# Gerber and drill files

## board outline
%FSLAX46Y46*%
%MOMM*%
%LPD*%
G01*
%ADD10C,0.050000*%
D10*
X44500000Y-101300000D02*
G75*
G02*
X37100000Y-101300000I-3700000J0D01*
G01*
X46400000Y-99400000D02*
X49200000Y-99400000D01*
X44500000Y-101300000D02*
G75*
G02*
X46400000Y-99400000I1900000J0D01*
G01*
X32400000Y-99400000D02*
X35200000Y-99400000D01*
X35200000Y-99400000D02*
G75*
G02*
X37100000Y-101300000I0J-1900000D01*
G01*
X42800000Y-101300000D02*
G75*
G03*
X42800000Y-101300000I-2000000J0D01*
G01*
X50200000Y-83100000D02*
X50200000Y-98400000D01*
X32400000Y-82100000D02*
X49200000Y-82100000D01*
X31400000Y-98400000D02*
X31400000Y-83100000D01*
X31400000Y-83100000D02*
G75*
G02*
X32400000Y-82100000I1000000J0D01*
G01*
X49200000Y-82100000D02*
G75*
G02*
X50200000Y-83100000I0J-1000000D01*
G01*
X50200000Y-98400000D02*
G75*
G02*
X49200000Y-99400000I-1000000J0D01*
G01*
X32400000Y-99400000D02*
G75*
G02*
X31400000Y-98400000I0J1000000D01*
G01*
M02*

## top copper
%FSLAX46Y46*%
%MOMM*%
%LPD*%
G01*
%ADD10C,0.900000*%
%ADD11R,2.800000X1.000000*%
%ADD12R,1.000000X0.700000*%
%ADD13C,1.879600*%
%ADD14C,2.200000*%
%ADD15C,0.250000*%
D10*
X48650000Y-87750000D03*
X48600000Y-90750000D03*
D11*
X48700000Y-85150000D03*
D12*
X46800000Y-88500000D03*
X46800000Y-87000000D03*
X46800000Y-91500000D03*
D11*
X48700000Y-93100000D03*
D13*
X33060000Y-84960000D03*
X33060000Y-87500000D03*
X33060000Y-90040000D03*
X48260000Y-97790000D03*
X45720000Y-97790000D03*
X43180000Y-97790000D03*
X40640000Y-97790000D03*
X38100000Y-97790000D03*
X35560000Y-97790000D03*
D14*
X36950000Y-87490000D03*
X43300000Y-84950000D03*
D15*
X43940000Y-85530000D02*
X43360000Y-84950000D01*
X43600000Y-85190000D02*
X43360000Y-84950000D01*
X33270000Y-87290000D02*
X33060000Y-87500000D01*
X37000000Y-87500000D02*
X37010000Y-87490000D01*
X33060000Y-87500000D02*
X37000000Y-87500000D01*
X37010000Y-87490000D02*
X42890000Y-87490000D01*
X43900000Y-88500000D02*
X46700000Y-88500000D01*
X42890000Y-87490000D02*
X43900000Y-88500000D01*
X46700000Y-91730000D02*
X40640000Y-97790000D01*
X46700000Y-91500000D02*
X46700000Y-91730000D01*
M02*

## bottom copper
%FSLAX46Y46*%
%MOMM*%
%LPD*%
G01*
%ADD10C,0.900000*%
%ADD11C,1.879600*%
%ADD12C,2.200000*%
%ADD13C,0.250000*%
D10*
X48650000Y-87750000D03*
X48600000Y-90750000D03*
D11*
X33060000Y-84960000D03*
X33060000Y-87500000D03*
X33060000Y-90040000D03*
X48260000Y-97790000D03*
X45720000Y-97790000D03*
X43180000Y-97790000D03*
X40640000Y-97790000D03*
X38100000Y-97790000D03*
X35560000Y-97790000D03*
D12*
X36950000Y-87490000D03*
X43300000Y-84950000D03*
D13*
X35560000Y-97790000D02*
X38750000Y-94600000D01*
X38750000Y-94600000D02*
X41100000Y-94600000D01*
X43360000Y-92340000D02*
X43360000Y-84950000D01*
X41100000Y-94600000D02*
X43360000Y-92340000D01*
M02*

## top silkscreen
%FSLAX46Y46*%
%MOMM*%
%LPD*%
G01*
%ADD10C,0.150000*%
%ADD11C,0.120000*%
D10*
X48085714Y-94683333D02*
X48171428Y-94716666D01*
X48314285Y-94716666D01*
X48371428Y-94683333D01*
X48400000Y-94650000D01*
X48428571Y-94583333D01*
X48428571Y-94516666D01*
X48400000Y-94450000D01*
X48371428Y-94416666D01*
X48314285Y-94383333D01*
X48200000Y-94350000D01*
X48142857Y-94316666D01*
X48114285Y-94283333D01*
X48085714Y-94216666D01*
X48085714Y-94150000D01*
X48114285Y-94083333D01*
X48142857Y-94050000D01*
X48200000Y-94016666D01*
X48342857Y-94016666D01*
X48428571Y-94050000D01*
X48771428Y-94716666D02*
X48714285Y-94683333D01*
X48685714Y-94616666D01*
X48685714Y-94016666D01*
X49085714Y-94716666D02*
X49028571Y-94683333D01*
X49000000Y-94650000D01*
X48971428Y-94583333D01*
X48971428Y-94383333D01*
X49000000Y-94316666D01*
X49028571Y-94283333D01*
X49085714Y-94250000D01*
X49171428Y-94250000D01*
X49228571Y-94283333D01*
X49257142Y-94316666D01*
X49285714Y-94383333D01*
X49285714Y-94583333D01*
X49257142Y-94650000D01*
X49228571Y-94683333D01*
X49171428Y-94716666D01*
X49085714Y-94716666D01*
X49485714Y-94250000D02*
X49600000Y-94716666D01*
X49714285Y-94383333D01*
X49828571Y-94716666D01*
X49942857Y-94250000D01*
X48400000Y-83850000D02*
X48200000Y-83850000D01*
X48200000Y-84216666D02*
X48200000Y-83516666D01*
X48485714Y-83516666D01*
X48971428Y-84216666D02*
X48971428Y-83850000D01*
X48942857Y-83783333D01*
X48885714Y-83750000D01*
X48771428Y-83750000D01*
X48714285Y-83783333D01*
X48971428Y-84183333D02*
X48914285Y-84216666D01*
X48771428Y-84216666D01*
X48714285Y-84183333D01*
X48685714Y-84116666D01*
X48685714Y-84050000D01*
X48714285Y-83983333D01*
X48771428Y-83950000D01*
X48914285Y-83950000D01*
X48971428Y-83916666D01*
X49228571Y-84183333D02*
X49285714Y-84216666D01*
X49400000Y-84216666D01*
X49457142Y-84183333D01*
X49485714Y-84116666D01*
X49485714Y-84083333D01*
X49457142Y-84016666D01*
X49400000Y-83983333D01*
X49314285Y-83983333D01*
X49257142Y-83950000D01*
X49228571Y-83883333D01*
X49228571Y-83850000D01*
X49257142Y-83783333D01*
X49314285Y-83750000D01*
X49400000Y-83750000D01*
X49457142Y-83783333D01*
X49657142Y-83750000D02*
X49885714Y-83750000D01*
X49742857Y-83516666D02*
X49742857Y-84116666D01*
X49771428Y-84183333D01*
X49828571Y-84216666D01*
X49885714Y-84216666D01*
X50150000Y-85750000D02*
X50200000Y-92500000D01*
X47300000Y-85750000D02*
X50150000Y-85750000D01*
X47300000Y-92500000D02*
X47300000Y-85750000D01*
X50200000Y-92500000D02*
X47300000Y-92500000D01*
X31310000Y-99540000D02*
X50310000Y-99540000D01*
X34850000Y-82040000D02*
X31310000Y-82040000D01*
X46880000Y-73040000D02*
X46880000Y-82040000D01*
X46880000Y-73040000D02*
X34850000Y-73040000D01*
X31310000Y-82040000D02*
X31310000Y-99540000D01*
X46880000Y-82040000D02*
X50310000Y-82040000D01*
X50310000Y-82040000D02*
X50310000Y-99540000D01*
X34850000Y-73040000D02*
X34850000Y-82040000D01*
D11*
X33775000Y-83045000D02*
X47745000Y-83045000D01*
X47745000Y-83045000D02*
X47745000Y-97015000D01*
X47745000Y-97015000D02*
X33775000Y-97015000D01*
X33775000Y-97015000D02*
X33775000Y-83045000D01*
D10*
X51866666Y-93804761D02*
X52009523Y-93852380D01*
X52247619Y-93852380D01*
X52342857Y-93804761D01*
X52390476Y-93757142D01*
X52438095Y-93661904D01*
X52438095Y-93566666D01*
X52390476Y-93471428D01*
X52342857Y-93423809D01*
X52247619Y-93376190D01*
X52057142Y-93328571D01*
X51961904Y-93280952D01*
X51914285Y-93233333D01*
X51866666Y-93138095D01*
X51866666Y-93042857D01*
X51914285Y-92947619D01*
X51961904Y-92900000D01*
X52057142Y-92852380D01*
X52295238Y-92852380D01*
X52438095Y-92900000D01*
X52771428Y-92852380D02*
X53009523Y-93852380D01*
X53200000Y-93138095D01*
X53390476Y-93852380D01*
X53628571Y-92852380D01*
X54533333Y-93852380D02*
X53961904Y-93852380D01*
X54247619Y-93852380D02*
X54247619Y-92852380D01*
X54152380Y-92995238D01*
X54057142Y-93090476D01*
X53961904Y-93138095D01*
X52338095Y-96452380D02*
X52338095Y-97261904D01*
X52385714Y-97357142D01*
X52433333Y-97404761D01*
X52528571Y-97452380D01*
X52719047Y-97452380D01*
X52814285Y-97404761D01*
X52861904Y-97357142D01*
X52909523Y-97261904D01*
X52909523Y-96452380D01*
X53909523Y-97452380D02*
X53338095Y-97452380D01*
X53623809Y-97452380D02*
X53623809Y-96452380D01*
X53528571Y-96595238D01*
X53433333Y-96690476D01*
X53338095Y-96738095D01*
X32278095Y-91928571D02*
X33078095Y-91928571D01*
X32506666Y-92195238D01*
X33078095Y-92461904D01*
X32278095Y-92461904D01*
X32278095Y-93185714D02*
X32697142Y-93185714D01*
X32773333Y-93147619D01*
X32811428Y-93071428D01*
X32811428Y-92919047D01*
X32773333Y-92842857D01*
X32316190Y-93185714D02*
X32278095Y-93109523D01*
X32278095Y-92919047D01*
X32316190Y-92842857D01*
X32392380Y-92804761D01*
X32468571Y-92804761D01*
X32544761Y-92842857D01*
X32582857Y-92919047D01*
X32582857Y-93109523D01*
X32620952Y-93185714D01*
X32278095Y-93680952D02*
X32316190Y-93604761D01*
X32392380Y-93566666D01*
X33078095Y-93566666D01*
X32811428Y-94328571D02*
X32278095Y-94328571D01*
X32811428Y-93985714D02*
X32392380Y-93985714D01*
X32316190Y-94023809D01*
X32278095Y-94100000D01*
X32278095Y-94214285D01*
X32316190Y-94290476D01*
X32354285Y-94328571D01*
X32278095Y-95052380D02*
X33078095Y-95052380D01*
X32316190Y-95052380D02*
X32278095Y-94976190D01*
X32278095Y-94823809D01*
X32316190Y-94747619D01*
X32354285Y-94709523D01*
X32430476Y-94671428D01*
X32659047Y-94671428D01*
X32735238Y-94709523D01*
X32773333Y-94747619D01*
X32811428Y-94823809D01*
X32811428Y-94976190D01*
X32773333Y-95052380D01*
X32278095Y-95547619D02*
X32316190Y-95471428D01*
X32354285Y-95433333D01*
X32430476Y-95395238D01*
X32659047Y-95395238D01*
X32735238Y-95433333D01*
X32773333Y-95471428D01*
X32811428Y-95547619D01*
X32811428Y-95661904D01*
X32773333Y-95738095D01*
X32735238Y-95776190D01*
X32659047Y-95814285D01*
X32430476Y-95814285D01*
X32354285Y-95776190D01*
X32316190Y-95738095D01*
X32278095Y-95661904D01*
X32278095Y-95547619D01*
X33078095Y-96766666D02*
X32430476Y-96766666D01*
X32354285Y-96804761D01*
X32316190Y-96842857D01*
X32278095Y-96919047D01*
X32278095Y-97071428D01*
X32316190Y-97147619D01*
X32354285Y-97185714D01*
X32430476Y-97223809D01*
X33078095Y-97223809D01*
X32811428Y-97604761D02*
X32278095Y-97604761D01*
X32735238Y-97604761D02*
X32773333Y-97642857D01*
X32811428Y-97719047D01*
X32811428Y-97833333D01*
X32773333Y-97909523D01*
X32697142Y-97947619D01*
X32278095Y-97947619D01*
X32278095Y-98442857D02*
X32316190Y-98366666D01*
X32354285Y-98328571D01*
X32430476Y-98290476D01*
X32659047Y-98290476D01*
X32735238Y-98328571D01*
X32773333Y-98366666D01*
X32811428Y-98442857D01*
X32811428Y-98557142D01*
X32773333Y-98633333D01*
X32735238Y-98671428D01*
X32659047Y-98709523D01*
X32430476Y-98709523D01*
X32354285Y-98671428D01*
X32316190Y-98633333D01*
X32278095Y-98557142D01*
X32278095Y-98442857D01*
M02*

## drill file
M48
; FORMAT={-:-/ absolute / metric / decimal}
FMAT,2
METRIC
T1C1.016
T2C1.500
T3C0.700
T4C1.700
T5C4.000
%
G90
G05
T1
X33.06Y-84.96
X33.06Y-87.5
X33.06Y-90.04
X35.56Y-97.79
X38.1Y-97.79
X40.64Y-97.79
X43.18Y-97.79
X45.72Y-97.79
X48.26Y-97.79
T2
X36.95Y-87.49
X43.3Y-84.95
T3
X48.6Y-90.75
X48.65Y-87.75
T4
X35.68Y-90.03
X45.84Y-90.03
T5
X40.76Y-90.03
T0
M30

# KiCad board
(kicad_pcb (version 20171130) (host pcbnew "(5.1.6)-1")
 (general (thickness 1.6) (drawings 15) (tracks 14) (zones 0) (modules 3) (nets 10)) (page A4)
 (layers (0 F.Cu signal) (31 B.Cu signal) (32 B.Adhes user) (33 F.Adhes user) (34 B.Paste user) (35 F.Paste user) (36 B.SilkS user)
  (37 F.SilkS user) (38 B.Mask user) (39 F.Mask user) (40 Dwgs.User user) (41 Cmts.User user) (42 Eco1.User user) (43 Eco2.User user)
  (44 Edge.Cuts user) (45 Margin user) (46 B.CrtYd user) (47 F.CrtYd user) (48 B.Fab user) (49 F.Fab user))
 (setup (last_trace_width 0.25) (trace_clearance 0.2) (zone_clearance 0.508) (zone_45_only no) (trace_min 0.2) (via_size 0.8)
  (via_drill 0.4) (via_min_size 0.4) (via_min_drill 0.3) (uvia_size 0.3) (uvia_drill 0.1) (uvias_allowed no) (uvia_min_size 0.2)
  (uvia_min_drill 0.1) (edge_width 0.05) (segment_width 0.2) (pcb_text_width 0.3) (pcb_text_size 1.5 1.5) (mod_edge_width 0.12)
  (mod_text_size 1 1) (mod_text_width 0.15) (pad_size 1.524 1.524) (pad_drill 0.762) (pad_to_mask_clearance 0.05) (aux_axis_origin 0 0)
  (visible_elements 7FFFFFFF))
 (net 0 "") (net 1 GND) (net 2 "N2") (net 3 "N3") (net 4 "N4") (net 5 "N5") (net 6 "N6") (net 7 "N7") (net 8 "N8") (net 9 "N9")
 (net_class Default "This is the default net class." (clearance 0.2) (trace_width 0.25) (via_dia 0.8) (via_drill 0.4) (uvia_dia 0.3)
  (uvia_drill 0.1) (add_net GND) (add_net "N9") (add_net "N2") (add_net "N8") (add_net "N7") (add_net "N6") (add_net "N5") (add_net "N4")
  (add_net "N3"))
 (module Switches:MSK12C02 (layer F.Cu) (at 50 93 180)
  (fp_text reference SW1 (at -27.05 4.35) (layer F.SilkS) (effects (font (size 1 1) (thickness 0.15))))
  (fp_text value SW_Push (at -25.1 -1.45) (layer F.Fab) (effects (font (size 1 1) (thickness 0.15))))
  (fp_line (start -0.2 0.5) (end 2.7 0.5) (layer F.SilkS) (width 0.15))
  (fp_line (start 2.7 0.5) (end 2.7 7.25) (layer F.SilkS) (width 0.15))
  (fp_line (start 2.7 7.25) (end -0.15 7.25) (layer F.SilkS) (width 0.15))
  (fp_line (start -0.15 7.25) (end -0.2 0.5) (layer F.SilkS) (width 0.15))
  (pad "" np_thru_hole circle (at 1.35 5.25 180) (size 0.9 0.9) (drill 0.7) (layers *.Cu *.Mask))
  (pad "" np_thru_hole circle (at 1.4 2.25 180) (size 0.9 0.9) (drill 0.7) (layers *.Cu *.Mask))
  (pad NC smd rect (at 1.3 7.85 180) (size 2.8 1) (layers F.Cu F.Paste F.Mask))
  (pad 2 smd rect (at 3.2 4.5 270) (size 0.7 1) (layers F.Cu F.Paste F.Mask) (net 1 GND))
  (pad 3 smd rect (at 3.2 6 270) (size 0.7 1) (layers F.Cu F.Paste F.Mask))
  (pad 1 smd rect (at 3.2 1.5 270) (size 0.7 1) (layers F.Cu F.Paste F.Mask) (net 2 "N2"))
  (pad NC smd rect (at 1.3 -0.1 180) (size 2.8 1) (layers F.Cu F.Paste F.Mask)))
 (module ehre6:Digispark (layer F.Cu) (at 41.91 97.79)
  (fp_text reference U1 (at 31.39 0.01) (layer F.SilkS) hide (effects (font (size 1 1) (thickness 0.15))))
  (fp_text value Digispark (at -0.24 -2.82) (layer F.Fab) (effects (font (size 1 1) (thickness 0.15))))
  (fp_line (start -7.06 -24.75) (end -7.06 -15.75) (layer F.SilkS) (width 0.15))
  (fp_line (start 8.4 -15.75) (end 8.4 1.75) (layer F.SilkS) (width 0.15))
  (fp_line (start 4.97 -15.75) (end 8.4 -15.75) (layer F.SilkS) (width 0.15))
  (fp_line (start -10.6 -15.75) (end -10.6 1.75) (layer F.SilkS) (width 0.15))
  (fp_line (start 4.97 -24.75) (end -7.06 -24.75) (layer F.SilkS) (width 0.15))
  (fp_line (start 4.97 -24.75) (end 4.97 -15.75) (layer F.SilkS) (width 0.15))
  (fp_line (start -7.06 -15.75) (end -10.6 -15.75) (layer F.SilkS) (width 0.15))
  (fp_line (start -10.6 1.75) (end 8.4 1.75) (layer F.SilkS) (width 0.15))
  (pad 9 thru_hole circle (at -8.85 -12.83) (size 1.8796 1.8796) (drill 1.016) (layers *.Cu *.Mask) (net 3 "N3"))
  (pad 8 thru_hole circle (at -8.85 -10.29) (size 1.8796 1.8796) (drill 1.016) (layers *.Cu *.Mask) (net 1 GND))
  (pad 7 thru_hole circle (at -8.85 -7.75) (size 1.8796 1.8796) (drill 1.016) (layers *.Cu *.Mask) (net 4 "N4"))
  (pad 6 thru_hole circle (at 6.35 0) (size 1.8796 1.8796) (drill 1.016) (layers *.Cu *.Mask) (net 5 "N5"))
  (pad 5 thru_hole circle (at 3.81 0) (size 1.8796 1.8796) (drill 1.016) (layers *.Cu *.Mask) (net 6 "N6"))
  (pad 4 thru_hole circle (at 1.27 0) (size 1.8796 1.8796) (drill 1.016) (layers *.Cu *.Mask) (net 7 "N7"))
  (pad 3 thru_hole circle (at -1.27 0) (size 1.8796 1.8796) (drill 1.016) (layers *.Cu *.Mask) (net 2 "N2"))
  (pad 2 thru_hole circle (at -3.81 0) (size 1.8796 1.8796) (drill 1.016) (layers *.Cu *.Mask) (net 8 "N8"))
  (pad 1 thru_hole circle (at -6.35 0) (size 1.8796 1.8796) (drill 1.016) (layers *.Cu *.Mask) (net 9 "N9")))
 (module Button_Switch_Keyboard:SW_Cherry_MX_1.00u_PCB (layer F.Cu) (at 43.3 84.95)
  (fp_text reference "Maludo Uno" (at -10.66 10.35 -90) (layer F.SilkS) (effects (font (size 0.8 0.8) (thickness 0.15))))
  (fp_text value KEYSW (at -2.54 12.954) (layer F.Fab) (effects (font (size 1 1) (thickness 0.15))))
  (fp_line (start -9.525 12.065) (end -9.525 -1.905) (layer F.SilkS) (width 0.12))
  (fp_line (start 4.445 12.065) (end -9.525 12.065) (layer F.SilkS) (width 0.12))
  (fp_line (start 4.445 -1.905) (end 4.445 12.065) (layer F.SilkS) (width 0.12))
  (fp_line (start -9.525 -1.905) (end 4.445 -1.905) (layer F.SilkS) (width 0.12))
  (pad "" np_thru_hole circle (at 2.54 5.08) (size 1.7 1.7) (drill 1.7) (layers *.Cu *.Mask))
  (pad "" np_thru_hole circle (at -7.62 5.08) (size 1.7 1.7) (drill 1.7) (layers *.Cu *.Mask))
  (pad "" np_thru_hole circle (at -2.54 5.08) (size 4 4) (drill 4) (layers *.Cu *.Mask))
  (pad 2 thru_hole circle (at -6.35 2.54) (size 2.2 2.2) (drill 1.5) (layers *.Cu *.Mask) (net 1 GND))
  (pad 1 thru_hole circle (at 0 0) (size 2.2 2.2) (drill 1.5) (layers *.Cu *.Mask) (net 9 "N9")))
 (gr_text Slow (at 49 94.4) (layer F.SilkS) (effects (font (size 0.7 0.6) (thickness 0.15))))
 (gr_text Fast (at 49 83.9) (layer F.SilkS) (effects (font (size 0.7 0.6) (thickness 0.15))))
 (gr_arc (start 40.8 101.3) (end 37.1 101.3) (angle -180) (layer Edge.Cuts) (width 0.05))
 (gr_line (start 46.4 99.4) (end 49.2 99.4) (layer Edge.Cuts) (width 0.05))
 (gr_arc (start 46.4 101.3) (end 46.4 99.4) (angle -90) (layer Edge.Cuts) (width 0.05))
 (gr_line (start 32.4 99.4) (end 35.2 99.4) (layer Edge.Cuts) (width 0.05))
 (gr_arc (start 35.2 101.3) (end 37.1 101.3) (angle -90) (layer Edge.Cuts) (width 0.05))
 (gr_circle (center 40.8 101.3) (end 42.8 101.3) (layer Edge.Cuts) (width 0.05))
 (gr_line (start 50.2 83.1) (end 50.2 98.4) (layer Edge.Cuts) (width 0.05))
 (gr_line (start 32.4 82.1) (end 49.2 82.1) (layer Edge.Cuts) (width 0.05))
 (gr_line (start 31.4 98.4) (end 31.4 83.1) (layer Edge.Cuts) (width 0.05))
 (gr_arc (start 32.4 83.1) (end 32.4 82.1) (angle -90) (layer Edge.Cuts) (width 0.05))
 (gr_arc (start 49.2 83.1) (end 50.2 83.1) (angle -90) (layer Edge.Cuts) (width 0.05))
 (gr_arc (start 49.2 98.4) (end 49.2 99.4) (angle -90) (layer Edge.Cuts) (width 0.05))
 (gr_arc (start 32.4 98.4) (end 31.4 98.4) (angle -90) (layer Edge.Cuts) (width 0.05))
 (segment (start 43.94 85.53) (end 43.36 84.95) (width 0.25) (layer F.Cu) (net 9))
 (segment (start 43.6 85.19) (end 43.36 84.95) (width 0.25) (layer F.Cu) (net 9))
 (segment (start 35.56 97.79) (end 38.75 94.6) (width 0.25) (layer B.Cu) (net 9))
 (segment (start 38.75 94.6) (end 41.1 94.6) (width 0.25) (layer B.Cu) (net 9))
 (segment (start 43.36 92.34) (end 43.36 84.95) (width 0.25) (layer B.Cu) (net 9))
 (segment (start 41.1 94.6) (end 43.36 92.34) (width 0.25) (layer B.Cu) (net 9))
 (segment (start 33.27 87.29) (end 33.06 87.5) (width 0.25) (layer F.Cu) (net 1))
 (segment (start 37 87.5) (end 37.01 87.49) (width 0.25) (layer F.Cu) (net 1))
 (segment (start 33.06 87.5) (end 37 87.5) (width 0.25) (layer F.Cu) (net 1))
 (segment (start 37.01 87.49) (end 42.89 87.49) (width 0.25) (layer F.Cu) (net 1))
 (segment (start 43.9 88.5) (end 46.7 88.5) (width 0.25) (layer F.Cu) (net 1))
 (segment (start 42.89 87.49) (end 43.9 88.5) (width 0.25) (layer F.Cu) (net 1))
 (segment (start 46.7 91.73) (end 40.64 97.79) (width 0.25) (layer F.Cu) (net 2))
 (segment (start 46.7 91.5) (end 46.7 91.73) (width 0.25) (layer F.Cu) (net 2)))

